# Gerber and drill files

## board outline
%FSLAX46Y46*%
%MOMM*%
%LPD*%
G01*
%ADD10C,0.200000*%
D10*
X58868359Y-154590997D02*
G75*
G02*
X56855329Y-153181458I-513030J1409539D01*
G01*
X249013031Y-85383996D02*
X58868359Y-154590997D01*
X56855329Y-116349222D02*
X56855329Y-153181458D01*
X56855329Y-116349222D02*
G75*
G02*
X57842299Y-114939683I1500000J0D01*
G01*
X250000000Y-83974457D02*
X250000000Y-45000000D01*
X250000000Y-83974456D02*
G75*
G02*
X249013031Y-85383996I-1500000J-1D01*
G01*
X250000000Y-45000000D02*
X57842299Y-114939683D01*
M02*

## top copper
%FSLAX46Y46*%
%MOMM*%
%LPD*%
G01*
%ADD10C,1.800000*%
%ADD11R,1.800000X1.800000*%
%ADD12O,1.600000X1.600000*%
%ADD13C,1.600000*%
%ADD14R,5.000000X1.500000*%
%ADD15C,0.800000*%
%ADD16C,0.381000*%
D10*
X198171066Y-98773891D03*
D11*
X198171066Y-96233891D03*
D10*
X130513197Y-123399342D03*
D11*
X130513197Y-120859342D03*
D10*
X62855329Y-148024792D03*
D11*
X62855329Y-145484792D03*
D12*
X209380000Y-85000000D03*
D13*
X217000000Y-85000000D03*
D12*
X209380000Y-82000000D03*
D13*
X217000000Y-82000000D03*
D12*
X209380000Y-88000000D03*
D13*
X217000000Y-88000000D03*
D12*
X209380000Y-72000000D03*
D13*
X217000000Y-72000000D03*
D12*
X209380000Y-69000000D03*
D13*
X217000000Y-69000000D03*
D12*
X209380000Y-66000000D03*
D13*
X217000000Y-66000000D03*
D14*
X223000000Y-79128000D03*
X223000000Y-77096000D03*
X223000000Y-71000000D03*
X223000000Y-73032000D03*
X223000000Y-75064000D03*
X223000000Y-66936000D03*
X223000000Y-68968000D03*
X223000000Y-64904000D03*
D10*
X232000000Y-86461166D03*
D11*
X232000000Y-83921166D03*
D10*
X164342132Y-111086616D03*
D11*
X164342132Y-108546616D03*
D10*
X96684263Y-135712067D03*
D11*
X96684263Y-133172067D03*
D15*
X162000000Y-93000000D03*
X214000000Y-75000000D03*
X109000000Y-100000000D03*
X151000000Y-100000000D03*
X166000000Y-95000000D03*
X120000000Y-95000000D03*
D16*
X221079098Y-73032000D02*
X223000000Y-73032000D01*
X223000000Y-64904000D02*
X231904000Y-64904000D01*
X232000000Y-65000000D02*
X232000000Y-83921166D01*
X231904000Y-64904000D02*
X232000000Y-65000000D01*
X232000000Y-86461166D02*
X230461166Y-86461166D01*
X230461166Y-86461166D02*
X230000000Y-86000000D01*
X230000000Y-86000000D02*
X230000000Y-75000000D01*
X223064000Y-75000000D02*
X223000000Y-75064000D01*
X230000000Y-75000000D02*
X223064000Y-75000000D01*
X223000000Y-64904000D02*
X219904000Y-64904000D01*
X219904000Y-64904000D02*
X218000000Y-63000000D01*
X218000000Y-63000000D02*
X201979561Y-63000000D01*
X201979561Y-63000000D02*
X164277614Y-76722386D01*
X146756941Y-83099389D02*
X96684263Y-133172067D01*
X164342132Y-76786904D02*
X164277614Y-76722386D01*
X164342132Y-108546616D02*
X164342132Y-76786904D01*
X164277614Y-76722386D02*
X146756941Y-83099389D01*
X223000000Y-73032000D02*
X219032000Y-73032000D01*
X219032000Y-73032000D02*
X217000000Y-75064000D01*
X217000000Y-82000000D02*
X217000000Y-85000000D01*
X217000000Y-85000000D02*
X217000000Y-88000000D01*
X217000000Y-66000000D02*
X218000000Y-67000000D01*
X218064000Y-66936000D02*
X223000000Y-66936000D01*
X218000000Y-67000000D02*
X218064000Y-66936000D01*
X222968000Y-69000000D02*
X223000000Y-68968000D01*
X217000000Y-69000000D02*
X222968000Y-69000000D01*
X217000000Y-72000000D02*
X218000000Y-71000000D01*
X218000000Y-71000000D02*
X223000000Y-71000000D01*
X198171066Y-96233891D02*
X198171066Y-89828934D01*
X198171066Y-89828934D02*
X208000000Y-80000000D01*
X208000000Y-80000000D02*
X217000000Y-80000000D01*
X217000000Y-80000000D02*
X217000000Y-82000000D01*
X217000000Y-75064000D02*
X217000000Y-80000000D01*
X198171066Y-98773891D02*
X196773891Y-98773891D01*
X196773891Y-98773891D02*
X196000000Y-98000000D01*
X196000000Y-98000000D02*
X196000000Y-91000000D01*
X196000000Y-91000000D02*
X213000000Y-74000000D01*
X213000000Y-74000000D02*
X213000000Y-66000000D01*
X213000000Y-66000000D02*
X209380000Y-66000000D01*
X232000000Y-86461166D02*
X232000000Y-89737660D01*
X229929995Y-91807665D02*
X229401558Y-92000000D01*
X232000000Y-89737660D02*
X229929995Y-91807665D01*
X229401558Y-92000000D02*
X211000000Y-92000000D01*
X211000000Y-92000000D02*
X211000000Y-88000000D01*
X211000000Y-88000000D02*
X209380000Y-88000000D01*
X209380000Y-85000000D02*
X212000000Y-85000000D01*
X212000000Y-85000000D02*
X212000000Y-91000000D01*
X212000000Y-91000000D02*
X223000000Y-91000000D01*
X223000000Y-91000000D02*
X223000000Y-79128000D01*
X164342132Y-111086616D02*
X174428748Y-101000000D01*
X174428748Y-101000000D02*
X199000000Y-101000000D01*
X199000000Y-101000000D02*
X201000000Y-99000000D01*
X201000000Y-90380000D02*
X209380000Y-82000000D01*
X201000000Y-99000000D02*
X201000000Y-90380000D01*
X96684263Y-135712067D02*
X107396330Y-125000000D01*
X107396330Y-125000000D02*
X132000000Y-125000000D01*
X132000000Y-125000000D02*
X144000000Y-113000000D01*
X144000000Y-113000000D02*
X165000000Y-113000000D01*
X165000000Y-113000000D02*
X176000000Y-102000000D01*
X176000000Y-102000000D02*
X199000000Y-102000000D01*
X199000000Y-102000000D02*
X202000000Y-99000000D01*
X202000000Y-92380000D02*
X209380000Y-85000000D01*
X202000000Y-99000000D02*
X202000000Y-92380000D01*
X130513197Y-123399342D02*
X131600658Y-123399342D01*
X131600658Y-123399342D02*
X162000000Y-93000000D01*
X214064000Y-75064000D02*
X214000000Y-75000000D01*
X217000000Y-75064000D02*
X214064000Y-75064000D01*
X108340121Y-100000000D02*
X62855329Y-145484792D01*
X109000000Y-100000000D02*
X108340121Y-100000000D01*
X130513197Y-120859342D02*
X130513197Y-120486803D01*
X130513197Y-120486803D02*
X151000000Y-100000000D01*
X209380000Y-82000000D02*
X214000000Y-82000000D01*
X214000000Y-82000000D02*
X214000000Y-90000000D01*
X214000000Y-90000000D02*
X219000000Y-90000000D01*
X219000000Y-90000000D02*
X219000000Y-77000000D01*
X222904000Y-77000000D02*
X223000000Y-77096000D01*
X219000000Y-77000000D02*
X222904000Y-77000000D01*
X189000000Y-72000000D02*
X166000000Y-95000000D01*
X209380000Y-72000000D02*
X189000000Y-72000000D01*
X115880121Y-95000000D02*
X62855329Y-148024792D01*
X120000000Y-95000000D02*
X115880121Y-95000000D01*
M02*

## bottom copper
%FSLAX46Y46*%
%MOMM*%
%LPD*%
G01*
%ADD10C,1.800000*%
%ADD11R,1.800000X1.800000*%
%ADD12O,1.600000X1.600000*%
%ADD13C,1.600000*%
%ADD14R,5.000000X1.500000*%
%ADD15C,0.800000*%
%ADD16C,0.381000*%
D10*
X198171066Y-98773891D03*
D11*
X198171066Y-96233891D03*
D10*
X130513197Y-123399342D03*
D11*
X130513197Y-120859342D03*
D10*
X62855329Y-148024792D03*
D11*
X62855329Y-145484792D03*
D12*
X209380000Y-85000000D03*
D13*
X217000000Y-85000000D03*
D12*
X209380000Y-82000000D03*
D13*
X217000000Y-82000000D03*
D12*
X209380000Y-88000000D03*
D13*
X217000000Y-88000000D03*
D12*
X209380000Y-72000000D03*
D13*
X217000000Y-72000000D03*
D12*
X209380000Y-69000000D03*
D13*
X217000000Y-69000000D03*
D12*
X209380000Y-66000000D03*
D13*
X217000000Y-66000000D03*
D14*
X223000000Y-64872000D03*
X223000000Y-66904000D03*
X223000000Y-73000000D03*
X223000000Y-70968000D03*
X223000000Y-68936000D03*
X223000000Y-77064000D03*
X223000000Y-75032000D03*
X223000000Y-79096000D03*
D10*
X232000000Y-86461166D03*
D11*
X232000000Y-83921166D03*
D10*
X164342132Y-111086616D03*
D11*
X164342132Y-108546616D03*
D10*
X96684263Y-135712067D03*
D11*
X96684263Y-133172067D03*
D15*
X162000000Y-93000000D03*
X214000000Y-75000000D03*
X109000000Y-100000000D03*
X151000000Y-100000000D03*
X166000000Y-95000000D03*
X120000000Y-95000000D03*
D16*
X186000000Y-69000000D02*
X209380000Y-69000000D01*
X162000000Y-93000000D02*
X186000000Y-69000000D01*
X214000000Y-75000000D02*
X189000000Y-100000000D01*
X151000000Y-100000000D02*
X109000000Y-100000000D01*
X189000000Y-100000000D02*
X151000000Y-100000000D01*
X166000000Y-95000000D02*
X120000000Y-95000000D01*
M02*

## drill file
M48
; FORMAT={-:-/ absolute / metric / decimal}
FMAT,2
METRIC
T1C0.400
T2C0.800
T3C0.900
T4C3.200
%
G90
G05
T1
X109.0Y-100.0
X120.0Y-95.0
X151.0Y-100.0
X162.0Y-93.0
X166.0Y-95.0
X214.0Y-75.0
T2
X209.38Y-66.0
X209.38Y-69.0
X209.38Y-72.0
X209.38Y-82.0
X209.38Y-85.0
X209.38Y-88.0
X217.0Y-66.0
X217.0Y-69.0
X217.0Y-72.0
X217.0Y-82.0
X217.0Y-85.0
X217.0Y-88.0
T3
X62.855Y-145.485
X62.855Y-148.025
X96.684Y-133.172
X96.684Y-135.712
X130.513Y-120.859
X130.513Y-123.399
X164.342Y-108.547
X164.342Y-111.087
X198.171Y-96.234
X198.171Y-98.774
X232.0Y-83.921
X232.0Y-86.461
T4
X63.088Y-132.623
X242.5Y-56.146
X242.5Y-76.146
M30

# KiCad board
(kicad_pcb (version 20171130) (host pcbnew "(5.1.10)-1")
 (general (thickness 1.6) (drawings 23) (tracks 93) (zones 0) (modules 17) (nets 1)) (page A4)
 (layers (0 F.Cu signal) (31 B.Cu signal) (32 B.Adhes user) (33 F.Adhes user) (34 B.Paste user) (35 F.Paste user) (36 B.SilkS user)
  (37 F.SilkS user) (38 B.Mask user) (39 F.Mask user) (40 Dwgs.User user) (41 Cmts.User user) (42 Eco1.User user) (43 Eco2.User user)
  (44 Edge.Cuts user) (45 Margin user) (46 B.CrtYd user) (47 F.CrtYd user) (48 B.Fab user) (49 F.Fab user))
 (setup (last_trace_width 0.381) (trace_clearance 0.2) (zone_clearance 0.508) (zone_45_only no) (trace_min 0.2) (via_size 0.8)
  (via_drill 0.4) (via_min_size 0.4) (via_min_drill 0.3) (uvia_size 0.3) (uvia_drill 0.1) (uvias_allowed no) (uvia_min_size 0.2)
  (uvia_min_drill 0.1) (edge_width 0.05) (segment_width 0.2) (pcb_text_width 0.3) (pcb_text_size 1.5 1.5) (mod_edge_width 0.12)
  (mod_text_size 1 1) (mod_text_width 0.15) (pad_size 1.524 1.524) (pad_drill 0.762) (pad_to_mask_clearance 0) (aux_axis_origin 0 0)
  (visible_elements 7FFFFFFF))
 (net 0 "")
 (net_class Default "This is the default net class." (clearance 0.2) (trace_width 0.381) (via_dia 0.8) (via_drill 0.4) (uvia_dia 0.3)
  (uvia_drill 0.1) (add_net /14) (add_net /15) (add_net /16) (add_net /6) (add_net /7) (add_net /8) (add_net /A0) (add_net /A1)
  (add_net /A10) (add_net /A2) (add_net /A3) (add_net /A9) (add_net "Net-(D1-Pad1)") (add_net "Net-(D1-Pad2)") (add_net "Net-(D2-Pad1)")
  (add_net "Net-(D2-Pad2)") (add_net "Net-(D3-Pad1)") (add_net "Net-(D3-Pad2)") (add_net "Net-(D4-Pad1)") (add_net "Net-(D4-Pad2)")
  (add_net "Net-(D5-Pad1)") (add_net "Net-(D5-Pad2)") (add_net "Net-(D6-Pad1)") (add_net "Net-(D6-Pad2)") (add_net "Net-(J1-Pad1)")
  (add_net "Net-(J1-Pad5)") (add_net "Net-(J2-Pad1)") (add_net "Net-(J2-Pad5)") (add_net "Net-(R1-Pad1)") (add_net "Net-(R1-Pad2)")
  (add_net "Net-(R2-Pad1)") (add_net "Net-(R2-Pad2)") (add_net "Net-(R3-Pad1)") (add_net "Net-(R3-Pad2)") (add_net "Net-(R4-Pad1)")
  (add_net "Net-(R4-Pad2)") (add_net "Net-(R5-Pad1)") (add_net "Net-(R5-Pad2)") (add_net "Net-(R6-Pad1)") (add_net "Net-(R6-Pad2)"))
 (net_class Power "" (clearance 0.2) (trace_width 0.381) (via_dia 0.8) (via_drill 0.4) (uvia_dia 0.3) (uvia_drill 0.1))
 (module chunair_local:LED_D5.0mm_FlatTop (layer F.Cu) (at 198.171066 96.233891 270)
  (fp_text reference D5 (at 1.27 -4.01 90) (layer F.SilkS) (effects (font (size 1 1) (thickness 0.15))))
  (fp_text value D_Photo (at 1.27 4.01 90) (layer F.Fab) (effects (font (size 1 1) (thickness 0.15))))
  (pad 2 thru_hole circle (at 2.54 0 270) (size 1.8 1.8) (drill 0.9) (layers *.Cu *.Mask))
  (pad 1 thru_hole rect (at 0 0 270) (size 1.8 1.8) (drill 0.9) (layers *.Cu *.Mask)))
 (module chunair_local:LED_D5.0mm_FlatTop (layer F.Cu) (at 130.513197 120.859342 270)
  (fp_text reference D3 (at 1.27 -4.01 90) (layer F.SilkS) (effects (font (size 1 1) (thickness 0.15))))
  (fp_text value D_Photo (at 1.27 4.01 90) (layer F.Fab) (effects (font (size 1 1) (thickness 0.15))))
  (pad 2 thru_hole circle (at 2.54 0 270) (size 1.8 1.8) (drill 0.9) (layers *.Cu *.Mask))
  (pad 1 thru_hole rect (at 0 0 270) (size 1.8 1.8) (drill 0.9) (layers *.Cu *.Mask)))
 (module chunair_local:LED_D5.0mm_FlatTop (layer F.Cu) (at 62.855329 145.484792 270)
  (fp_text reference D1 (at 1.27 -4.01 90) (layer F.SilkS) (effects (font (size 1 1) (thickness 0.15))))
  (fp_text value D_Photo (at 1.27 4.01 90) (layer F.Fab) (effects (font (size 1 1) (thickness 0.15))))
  (pad 2 thru_hole circle (at 2.54 0 270) (size 1.8 1.8) (drill 0.9) (layers *.Cu *.Mask))
  (pad 1 thru_hole rect (at 0 0 270) (size 1.8 1.8) (drill 0.9) (layers *.Cu *.Mask)))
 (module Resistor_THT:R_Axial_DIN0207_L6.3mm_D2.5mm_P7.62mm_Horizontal (layer F.Cu) (at 217 85 180)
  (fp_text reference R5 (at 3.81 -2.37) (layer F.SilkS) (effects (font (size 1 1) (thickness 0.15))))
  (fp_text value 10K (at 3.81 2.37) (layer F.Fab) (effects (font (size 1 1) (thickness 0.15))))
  (pad 2 thru_hole oval (at 7.62 0 180) (size 1.6 1.6) (drill 0.8) (layers *.Cu *.Mask))
  (pad 1 thru_hole circle (at 0 0 180) (size 1.6 1.6) (drill 0.8) (layers *.Cu *.Mask)))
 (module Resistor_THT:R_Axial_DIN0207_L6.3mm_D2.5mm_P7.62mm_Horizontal (layer F.Cu) (at 217 82 180)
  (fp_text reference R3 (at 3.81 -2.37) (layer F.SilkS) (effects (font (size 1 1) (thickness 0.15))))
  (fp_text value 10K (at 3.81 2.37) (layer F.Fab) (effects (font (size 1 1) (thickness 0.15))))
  (pad 2 thru_hole oval (at 7.62 0 180) (size 1.6 1.6) (drill 0.8) (layers *.Cu *.Mask))
  (pad 1 thru_hole circle (at 0 0 180) (size 1.6 1.6) (drill 0.8) (layers *.Cu *.Mask)))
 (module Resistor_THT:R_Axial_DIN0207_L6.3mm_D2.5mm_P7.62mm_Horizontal (layer F.Cu) (at 217 88 180)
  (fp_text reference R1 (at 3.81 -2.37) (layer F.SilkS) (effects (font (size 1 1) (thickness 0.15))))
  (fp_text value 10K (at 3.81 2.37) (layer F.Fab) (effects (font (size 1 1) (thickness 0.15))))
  (pad 2 thru_hole oval (at 7.62 0 180) (size 1.6 1.6) (drill 0.8) (layers *.Cu *.Mask))
  (pad 1 thru_hole circle (at 0 0 180) (size 1.6 1.6) (drill 0.8) (layers *.Cu *.Mask)))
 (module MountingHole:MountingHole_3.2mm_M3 (layer F.Cu) (at 242.5 56.145894)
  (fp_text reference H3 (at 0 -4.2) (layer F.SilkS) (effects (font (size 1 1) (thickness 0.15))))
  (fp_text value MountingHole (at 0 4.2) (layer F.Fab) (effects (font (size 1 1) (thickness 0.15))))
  (pad 1 np_thru_hole circle (at 0 0) (size 3.2 3.2) (drill 3.2) (layers *.Cu *.Mask)))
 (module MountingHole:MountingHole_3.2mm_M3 (layer F.Cu) (at 242.5 76.145894)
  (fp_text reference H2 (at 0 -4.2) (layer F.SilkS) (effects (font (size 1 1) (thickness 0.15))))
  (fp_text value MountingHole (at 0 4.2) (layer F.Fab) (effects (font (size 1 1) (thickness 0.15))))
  (pad 1 np_thru_hole circle (at 0 0) (size 3.2 3.2) (drill 3.2) (layers *.Cu *.Mask)))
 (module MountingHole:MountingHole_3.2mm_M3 (layer F.Cu) (at 63.08849 132.623118)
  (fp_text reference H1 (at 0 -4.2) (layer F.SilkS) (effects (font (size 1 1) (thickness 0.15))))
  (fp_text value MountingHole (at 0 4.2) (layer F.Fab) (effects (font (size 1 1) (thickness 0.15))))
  (pad 1 np_thru_hole circle (at 0 0) (size 3.2 3.2) (drill 3.2) (layers *.Cu *.Mask)))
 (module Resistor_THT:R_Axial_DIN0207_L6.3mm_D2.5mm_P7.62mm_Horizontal (layer F.Cu) (at 217 72 180)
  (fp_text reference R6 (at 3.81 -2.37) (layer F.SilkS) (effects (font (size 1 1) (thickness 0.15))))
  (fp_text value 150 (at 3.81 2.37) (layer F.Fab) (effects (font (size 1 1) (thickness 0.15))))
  (pad 2 thru_hole oval (at 7.62 0 180) (size 1.6 1.6) (drill 0.8) (layers *.Cu *.Mask))
  (pad 1 thru_hole circle (at 0 0 180) (size 1.6 1.6) (drill 0.8) (layers *.Cu *.Mask)))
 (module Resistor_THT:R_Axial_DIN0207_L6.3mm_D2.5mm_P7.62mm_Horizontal (layer F.Cu) (at 217 69 180)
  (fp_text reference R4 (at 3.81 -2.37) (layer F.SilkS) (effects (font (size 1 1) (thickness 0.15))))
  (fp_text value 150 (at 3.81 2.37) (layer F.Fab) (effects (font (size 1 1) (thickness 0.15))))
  (pad 2 thru_hole oval (at 7.62 0 180) (size 1.6 1.6) (drill 0.8) (layers *.Cu *.Mask))
  (pad 1 thru_hole circle (at 0 0 180) (size 1.6 1.6) (drill 0.8) (layers *.Cu *.Mask)))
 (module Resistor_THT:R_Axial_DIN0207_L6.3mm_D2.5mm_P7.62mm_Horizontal (layer F.Cu) (at 217 66 180)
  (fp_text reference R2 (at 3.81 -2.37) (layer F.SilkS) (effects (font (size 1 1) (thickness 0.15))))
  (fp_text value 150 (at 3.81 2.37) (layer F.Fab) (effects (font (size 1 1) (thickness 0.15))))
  (pad 2 thru_hole oval (at 7.62 0 180) (size 1.6 1.6) (drill 0.8) (layers *.Cu *.Mask))
  (pad 1 thru_hole circle (at 0 0 180) (size 1.6 1.6) (drill 0.8) (layers *.Cu *.Mask)))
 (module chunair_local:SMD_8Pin (layer B.Cu) (at 223 73)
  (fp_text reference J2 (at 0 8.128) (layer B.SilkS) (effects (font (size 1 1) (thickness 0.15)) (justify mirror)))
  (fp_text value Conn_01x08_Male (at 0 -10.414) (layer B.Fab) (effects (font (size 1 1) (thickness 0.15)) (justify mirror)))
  (pad 8 smd rect (at 0 -8.128) (size 5 1.5) (layers B.Cu B.Paste B.Mask))
  (pad 7 smd rect (at 0 -6.096) (size 5 1.5) (layers B.Cu B.Paste B.Mask))
  (pad 4 smd rect (at 0 0) (size 5 1.5) (layers B.Cu B.Paste B.Mask))
  (pad 5 smd rect (at 0 -2.032) (size 5 1.5) (layers B.Cu B.Paste B.Mask))
  (pad 6 smd rect (at 0 -4.064) (size 5 1.5) (layers B.Cu B.Paste B.Mask))
  (pad 2 smd rect (at 0 4.064) (size 5 1.5) (layers B.Cu B.Paste B.Mask))
  (pad 3 smd rect (at 0 2.032) (size 5 1.5) (layers B.Cu B.Paste B.Mask))
  (pad 1 smd rect (at 0 6.096) (size 5 1.5) (layers B.Cu B.Paste B.Mask)))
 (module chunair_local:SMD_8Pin (layer F.Cu) (at 223 71)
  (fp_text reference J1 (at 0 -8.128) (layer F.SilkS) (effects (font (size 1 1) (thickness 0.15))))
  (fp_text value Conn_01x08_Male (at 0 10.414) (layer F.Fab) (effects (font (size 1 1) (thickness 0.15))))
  (pad 8 smd rect (at 0 8.128) (size 5 1.5) (layers F.Cu F.Paste F.Mask))
  (pad 7 smd rect (at 0 6.096) (size 5 1.5) (layers F.Cu F.Paste F.Mask))
  (pad 4 smd rect (at 0 0) (size 5 1.5) (layers F.Cu F.Paste F.Mask))
  (pad 5 smd rect (at 0 2.032) (size 5 1.5) (layers F.Cu F.Paste F.Mask))
  (pad 6 smd rect (at 0 4.064) (size 5 1.5) (layers F.Cu F.Paste F.Mask))
  (pad 2 smd rect (at 0 -4.064) (size 5 1.5) (layers F.Cu F.Paste F.Mask))
  (pad 3 smd rect (at 0 -2.032) (size 5 1.5) (layers F.Cu F.Paste F.Mask))
  (pad 1 smd rect (at 0 -6.096) (size 5 1.5) (layers F.Cu F.Paste F.Mask)))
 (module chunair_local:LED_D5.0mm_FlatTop (layer B.Cu) (at 232 83.921166 270)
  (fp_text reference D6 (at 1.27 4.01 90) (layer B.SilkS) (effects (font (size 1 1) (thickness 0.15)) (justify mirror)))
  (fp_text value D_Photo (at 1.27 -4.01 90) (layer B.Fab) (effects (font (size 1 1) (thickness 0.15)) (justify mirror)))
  (pad 2 thru_hole circle (at 2.54 0 270) (size 1.8 1.8) (drill 0.9) (layers *.Cu *.Mask))
  (pad 1 thru_hole rect (at 0 0 270) (size 1.8 1.8) (drill 0.9) (layers *.Cu *.Mask)))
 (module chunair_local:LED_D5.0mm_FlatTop (layer B.Cu) (at 164.342132 108.546616 270)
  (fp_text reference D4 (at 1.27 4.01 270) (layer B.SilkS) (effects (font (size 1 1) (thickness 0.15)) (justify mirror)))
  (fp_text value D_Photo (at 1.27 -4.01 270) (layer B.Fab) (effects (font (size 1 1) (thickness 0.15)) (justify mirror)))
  (pad 2 thru_hole circle (at 2.54 0 270) (size 1.8 1.8) (drill 0.9) (layers *.Cu *.Mask))
  (pad 1 thru_hole rect (at 0 0 270) (size 1.8 1.8) (drill 0.9) (layers *.Cu *.Mask)))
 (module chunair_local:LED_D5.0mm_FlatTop (layer B.Cu) (at 96.684263 133.172067 270)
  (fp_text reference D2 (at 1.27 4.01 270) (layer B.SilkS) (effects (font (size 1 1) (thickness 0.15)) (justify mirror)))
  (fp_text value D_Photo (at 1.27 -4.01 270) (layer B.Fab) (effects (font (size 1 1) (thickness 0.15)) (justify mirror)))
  (pad 2 thru_hole circle (at 2.54 0 270) (size 1.8 1.8) (drill 0.9) (layers *.Cu *.Mask))
  (pad 1 thru_hole rect (at 0 0 270) (size 1.8 1.8) (drill 0.9) (layers *.Cu *.Mask)))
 (gr_arc (start 58.355329 153.181458) (end 56.855329 153.181458) (angle -110) (layer Edge.Cuts) (width 0.2))
 (gr_line (start 249.013031 85.383996) (end 58.868359 154.590997) (layer Edge.Cuts) (width 0.2))
 (gr_line (start 56.855329 116.349222) (end 56.855329 153.181458) (layer Edge.Cuts) (width 0.2))
 (gr_arc (start 58.355329 116.349222) (end 57.842299 114.939683) (angle -70) (layer Edge.Cuts) (width 0.2))
 (gr_line (start 250 83.974457) (end 250 45) (layer Edge.Cuts) (width 0.2))
 (gr_arc (start 248.5 83.974457) (end 249.013031 85.383996) (angle -70) (layer Edge.Cuts) (width 0.2))
 (gr_line (start 250 45) (end 57.842299 114.939683) (layer Edge.Cuts) (width 0.2))
 (segment (start 221.079098 73.032) (end 223 73.032) (width 0.381) (layer F.Cu) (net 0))
 (segment (start 223 64.904) (end 231.904 64.904) (width 0.381) (layer F.Cu) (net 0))
 (segment (start 232 65) (end 232 83.921166) (width 0.381) (layer F.Cu) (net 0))
 (segment (start 231.904 64.904) (end 232 65) (width 0.381) (layer F.Cu) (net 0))
 (segment (start 232 86.461166) (end 230.461166 86.461166) (width 0.381) (layer F.Cu) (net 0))
 (segment (start 230.461166 86.461166) (end 230 86) (width 0.381) (layer F.Cu) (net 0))
 (segment (start 230 86) (end 230 75) (width 0.381) (layer F.Cu) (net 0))
 (segment (start 223.064 75) (end 223 75.064) (width 0.381) (layer F.Cu) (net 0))
 (segment (start 230 75) (end 223.064 75) (width 0.381) (layer F.Cu) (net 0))
 (segment (start 223 64.904) (end 219.904 64.904) (width 0.381) (layer F.Cu) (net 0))
 (segment (start 219.904 64.904) (end 218 63) (width 0.381) (layer F.Cu) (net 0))
 (segment (start 218 63) (end 201.979561 63) (width 0.381) (layer F.Cu) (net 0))
 (segment (start 201.979561 63) (end 164.277614 76.722386) (width 0.381) (layer F.Cu) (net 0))
 (segment (start 146.756941 83.099389) (end 96.684263 133.172067) (width 0.381) (layer F.Cu) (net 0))
 (segment (start 164.342132 76.786904) (end 164.277614 76.722386) (width 0.381) (layer F.Cu) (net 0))
 (segment (start 164.342132 108.546616) (end 164.342132 76.786904) (width 0.381) (layer F.Cu) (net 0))
 (segment (start 164.277614 76.722386) (end 146.756941 83.099389) (width 0.381) (layer F.Cu) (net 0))
 (segment (start 223 73.032) (end 219.032 73.032) (width 0.381) (layer F.Cu) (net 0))
 (segment (start 219.032 73.032) (end 217 75.064) (width 0.381) (layer F.Cu) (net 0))
 (segment (start 217 82) (end 217 85) (width 0.381) (layer F.Cu) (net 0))
 (segment (start 217 85) (end 217 88) (width 0.381) (layer F.Cu) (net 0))
 (segment (start 217 66) (end 218 67) (width 0.381) (layer F.Cu) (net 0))
 (segment (start 218.064 66.936) (end 223 66.936) (width 0.381) (layer F.Cu) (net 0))
 (segment (start 218 67) (end 218.064 66.936) (width 0.381) (layer F.Cu) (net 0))
 (segment (start 222.968 69) (end 223 68.968) (width 0.381) (layer F.Cu) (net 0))
 (segment (start 217 69) (end 222.968 69) (width 0.381) (layer F.Cu) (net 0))
 (segment (start 217 72) (end 218 71) (width 0.381) (layer F.Cu) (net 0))
 (segment (start 218 71) (end 223 71) (width 0.381) (layer F.Cu) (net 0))
 (segment (start 198.171066 96.233891) (end 198.171066 89.828934) (width 0.381) (layer F.Cu) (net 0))
 (segment (start 198.171066 89.828934) (end 208 80) (width 0.381) (layer F.Cu) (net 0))
 (segment (start 208 80) (end 217 80) (width 0.381) (layer F.Cu) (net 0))
 (segment (start 217 80) (end 217 82) (width 0.381) (layer F.Cu) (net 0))
 (segment (start 217 75.064) (end 217 80) (width 0.381) (layer F.Cu) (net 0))
 (segment (start 198.171066 98.773891) (end 196.773891 98.773891) (width 0.381) (layer F.Cu) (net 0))
 (segment (start 196.773891 98.773891) (end 196 98) (width 0.381) (layer F.Cu) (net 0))
 (segment (start 196 98) (end 196 91) (width 0.381) (layer F.Cu) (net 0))
 (segment (start 196 91) (end 213 74) (width 0.381) (layer F.Cu) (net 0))
 (segment (start 213 74) (end 213 66) (width 0.381) (layer F.Cu) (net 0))
 (segment (start 213 66) (end 209.38 66) (width 0.381) (layer F.Cu) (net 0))
 (segment (start 232 86.461166) (end 232 89.73766) (width 0.381) (layer F.Cu) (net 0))
 (segment (start 229.929995 91.807665) (end 229.401558 92) (width 0.381) (layer F.Cu) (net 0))
 (segment (start 232 89.73766) (end 229.929995 91.807665) (width 0.381) (layer F.Cu) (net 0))
 (segment (start 229.401558 92) (end 211 92) (width 0.381) (layer F.Cu) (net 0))
 (segment (start 211 92) (end 211 88) (width 0.381) (layer F.Cu) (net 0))
 (segment (start 211 88) (end 209.38 88) (width 0.381) (layer F.Cu) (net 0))
 (segment (start 209.38 85) (end 212 85) (width 0.381) (layer F.Cu) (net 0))
 (segment (start 212 85) (end 212 91) (width 0.381) (layer F.Cu) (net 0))
 (segment (start 212 91) (end 223 91) (width 0.381) (layer F.Cu) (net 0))
 (segment (start 223 91) (end 223 79.128) (width 0.381) (layer F.Cu) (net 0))
 (segment (start 164.342132 111.086616) (end 174.428748 101) (width 0.381) (layer F.Cu) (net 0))
 (segment (start 174.428748 101) (end 199 101) (width 0.381) (layer F.Cu) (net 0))
 (segment (start 199 101) (end 201 99) (width 0.381) (layer F.Cu) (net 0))
 (segment (start 201 90.38) (end 209.38 82) (width 0.381) (layer F.Cu) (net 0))
 (segment (start 201 99) (end 201 90.38) (width 0.381) (layer F.Cu) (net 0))
 (segment (start 96.684263 135.712067) (end 107.39633 125) (width 0.381) (layer F.Cu) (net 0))
 (segment (start 107.39633 125) (end 132 125) (width 0.381) (layer F.Cu) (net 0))
 (segment (start 132 125) (end 144 113) (width 0.381) (layer F.Cu) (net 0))
 (segment (start 144 113) (end 165 113) (width 0.381) (layer F.Cu) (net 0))
 (segment (start 165 113) (end 176 102) (width 0.381) (layer F.Cu) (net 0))
 (segment (start 176 102) (end 199 102) (width 0.381) (layer F.Cu) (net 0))
 (segment (start 199 102) (end 202 99) (width 0.381) (layer F.Cu) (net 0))
 (segment (start 202 92.38) (end 209.38 85) (width 0.381) (layer F.Cu) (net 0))
 (segment (start 202 99) (end 202 92.38) (width 0.381) (layer F.Cu) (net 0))
 (segment (start 130.513197 123.399342) (end 131.600658 123.399342) (width 0.381) (layer F.Cu) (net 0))
 (via (at 162 93) (size 0.8) (drill 0.4) (layers F.Cu B.Cu) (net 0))
 (segment (start 131.600658 123.399342) (end 162 93) (width 0.381) (layer F.Cu) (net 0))
 (segment (start 186 69) (end 209.38 69) (width 0.381) (layer B.Cu) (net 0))
 (segment (start 162 93) (end 186 69) (width 0.381) (layer B.Cu) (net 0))
 (via (at 214 75) (size 0.8) (drill 0.4) (layers F.Cu B.Cu) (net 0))
 (segment (start 214.064 75.064) (end 214 75) (width 0.381) (layer F.Cu) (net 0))
 (segment (start 217 75.064) (end 214.064 75.064) (width 0.381) (layer F.Cu) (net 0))
 (via (at 109 100) (size 0.8) (drill 0.4) (layers F.Cu B.Cu) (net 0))
 (segment (start 214 75) (end 189 100) (width 0.381) (layer B.Cu) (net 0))
 (segment (start 108.340121 100) (end 62.855329 145.484792) (width 0.381) (layer F.Cu) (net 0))
 (segment (start 109 100) (end 108.340121 100) (width 0.381) (layer F.Cu) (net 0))
 (segment (start 130.513197 120.859342) (end 130.513197 120.486803) (width 0.381) (layer F.Cu) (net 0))
 (via (at 151 100) (size 0.8) (drill 0.4) (layers F.Cu B.Cu) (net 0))
 (segment (start 130.513197 120.486803) (end 151 100) (width 0.381) (layer F.Cu) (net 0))
 (segment (start 151 100) (end 109 100) (width 0.381) (layer B.Cu) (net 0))
 (segment (start 189 100) (end 151 100) (width 0.381) (layer B.Cu) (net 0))
 (segment (start 209.38 82) (end 214 82) (width 0.381) (layer F.Cu) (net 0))
 (segment (start 214 82) (end 214 90) (width 0.381) (layer F.Cu) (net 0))
 (segment (start 214 90) (end 219 90) (width 0.381) (layer F.Cu) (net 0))
 (segment (start 219 90) (end 219 77) (width 0.381) (layer F.Cu) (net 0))
 (segment (start 222.904 77) (end 223 77.096) (width 0.381) (layer F.Cu) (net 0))
 (segment (start 219 77) (end 222.904 77) (width 0.381) (layer F.Cu) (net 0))
 (via (at 166 95) (size 0.8) (drill 0.4) (layers F.Cu B.Cu) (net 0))
 (segment (start 189 72) (end 166 95) (width 0.381) (layer F.Cu) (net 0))
 (segment (start 209.38 72) (end 189 72) (width 0.381) (layer F.Cu) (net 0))
 (via (at 120 95) (size 0.8) (drill 0.4) (layers F.Cu B.Cu) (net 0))
 (segment (start 166 95) (end 120 95) (width 0.381) (layer B.Cu) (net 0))
 (segment (start 115.880121 95) (end 62.855329 148.024792) (width 0.381) (layer F.Cu) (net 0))
 (segment (start 120 95) (end 115.880121 95) (width 0.381) (layer F.Cu) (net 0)))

